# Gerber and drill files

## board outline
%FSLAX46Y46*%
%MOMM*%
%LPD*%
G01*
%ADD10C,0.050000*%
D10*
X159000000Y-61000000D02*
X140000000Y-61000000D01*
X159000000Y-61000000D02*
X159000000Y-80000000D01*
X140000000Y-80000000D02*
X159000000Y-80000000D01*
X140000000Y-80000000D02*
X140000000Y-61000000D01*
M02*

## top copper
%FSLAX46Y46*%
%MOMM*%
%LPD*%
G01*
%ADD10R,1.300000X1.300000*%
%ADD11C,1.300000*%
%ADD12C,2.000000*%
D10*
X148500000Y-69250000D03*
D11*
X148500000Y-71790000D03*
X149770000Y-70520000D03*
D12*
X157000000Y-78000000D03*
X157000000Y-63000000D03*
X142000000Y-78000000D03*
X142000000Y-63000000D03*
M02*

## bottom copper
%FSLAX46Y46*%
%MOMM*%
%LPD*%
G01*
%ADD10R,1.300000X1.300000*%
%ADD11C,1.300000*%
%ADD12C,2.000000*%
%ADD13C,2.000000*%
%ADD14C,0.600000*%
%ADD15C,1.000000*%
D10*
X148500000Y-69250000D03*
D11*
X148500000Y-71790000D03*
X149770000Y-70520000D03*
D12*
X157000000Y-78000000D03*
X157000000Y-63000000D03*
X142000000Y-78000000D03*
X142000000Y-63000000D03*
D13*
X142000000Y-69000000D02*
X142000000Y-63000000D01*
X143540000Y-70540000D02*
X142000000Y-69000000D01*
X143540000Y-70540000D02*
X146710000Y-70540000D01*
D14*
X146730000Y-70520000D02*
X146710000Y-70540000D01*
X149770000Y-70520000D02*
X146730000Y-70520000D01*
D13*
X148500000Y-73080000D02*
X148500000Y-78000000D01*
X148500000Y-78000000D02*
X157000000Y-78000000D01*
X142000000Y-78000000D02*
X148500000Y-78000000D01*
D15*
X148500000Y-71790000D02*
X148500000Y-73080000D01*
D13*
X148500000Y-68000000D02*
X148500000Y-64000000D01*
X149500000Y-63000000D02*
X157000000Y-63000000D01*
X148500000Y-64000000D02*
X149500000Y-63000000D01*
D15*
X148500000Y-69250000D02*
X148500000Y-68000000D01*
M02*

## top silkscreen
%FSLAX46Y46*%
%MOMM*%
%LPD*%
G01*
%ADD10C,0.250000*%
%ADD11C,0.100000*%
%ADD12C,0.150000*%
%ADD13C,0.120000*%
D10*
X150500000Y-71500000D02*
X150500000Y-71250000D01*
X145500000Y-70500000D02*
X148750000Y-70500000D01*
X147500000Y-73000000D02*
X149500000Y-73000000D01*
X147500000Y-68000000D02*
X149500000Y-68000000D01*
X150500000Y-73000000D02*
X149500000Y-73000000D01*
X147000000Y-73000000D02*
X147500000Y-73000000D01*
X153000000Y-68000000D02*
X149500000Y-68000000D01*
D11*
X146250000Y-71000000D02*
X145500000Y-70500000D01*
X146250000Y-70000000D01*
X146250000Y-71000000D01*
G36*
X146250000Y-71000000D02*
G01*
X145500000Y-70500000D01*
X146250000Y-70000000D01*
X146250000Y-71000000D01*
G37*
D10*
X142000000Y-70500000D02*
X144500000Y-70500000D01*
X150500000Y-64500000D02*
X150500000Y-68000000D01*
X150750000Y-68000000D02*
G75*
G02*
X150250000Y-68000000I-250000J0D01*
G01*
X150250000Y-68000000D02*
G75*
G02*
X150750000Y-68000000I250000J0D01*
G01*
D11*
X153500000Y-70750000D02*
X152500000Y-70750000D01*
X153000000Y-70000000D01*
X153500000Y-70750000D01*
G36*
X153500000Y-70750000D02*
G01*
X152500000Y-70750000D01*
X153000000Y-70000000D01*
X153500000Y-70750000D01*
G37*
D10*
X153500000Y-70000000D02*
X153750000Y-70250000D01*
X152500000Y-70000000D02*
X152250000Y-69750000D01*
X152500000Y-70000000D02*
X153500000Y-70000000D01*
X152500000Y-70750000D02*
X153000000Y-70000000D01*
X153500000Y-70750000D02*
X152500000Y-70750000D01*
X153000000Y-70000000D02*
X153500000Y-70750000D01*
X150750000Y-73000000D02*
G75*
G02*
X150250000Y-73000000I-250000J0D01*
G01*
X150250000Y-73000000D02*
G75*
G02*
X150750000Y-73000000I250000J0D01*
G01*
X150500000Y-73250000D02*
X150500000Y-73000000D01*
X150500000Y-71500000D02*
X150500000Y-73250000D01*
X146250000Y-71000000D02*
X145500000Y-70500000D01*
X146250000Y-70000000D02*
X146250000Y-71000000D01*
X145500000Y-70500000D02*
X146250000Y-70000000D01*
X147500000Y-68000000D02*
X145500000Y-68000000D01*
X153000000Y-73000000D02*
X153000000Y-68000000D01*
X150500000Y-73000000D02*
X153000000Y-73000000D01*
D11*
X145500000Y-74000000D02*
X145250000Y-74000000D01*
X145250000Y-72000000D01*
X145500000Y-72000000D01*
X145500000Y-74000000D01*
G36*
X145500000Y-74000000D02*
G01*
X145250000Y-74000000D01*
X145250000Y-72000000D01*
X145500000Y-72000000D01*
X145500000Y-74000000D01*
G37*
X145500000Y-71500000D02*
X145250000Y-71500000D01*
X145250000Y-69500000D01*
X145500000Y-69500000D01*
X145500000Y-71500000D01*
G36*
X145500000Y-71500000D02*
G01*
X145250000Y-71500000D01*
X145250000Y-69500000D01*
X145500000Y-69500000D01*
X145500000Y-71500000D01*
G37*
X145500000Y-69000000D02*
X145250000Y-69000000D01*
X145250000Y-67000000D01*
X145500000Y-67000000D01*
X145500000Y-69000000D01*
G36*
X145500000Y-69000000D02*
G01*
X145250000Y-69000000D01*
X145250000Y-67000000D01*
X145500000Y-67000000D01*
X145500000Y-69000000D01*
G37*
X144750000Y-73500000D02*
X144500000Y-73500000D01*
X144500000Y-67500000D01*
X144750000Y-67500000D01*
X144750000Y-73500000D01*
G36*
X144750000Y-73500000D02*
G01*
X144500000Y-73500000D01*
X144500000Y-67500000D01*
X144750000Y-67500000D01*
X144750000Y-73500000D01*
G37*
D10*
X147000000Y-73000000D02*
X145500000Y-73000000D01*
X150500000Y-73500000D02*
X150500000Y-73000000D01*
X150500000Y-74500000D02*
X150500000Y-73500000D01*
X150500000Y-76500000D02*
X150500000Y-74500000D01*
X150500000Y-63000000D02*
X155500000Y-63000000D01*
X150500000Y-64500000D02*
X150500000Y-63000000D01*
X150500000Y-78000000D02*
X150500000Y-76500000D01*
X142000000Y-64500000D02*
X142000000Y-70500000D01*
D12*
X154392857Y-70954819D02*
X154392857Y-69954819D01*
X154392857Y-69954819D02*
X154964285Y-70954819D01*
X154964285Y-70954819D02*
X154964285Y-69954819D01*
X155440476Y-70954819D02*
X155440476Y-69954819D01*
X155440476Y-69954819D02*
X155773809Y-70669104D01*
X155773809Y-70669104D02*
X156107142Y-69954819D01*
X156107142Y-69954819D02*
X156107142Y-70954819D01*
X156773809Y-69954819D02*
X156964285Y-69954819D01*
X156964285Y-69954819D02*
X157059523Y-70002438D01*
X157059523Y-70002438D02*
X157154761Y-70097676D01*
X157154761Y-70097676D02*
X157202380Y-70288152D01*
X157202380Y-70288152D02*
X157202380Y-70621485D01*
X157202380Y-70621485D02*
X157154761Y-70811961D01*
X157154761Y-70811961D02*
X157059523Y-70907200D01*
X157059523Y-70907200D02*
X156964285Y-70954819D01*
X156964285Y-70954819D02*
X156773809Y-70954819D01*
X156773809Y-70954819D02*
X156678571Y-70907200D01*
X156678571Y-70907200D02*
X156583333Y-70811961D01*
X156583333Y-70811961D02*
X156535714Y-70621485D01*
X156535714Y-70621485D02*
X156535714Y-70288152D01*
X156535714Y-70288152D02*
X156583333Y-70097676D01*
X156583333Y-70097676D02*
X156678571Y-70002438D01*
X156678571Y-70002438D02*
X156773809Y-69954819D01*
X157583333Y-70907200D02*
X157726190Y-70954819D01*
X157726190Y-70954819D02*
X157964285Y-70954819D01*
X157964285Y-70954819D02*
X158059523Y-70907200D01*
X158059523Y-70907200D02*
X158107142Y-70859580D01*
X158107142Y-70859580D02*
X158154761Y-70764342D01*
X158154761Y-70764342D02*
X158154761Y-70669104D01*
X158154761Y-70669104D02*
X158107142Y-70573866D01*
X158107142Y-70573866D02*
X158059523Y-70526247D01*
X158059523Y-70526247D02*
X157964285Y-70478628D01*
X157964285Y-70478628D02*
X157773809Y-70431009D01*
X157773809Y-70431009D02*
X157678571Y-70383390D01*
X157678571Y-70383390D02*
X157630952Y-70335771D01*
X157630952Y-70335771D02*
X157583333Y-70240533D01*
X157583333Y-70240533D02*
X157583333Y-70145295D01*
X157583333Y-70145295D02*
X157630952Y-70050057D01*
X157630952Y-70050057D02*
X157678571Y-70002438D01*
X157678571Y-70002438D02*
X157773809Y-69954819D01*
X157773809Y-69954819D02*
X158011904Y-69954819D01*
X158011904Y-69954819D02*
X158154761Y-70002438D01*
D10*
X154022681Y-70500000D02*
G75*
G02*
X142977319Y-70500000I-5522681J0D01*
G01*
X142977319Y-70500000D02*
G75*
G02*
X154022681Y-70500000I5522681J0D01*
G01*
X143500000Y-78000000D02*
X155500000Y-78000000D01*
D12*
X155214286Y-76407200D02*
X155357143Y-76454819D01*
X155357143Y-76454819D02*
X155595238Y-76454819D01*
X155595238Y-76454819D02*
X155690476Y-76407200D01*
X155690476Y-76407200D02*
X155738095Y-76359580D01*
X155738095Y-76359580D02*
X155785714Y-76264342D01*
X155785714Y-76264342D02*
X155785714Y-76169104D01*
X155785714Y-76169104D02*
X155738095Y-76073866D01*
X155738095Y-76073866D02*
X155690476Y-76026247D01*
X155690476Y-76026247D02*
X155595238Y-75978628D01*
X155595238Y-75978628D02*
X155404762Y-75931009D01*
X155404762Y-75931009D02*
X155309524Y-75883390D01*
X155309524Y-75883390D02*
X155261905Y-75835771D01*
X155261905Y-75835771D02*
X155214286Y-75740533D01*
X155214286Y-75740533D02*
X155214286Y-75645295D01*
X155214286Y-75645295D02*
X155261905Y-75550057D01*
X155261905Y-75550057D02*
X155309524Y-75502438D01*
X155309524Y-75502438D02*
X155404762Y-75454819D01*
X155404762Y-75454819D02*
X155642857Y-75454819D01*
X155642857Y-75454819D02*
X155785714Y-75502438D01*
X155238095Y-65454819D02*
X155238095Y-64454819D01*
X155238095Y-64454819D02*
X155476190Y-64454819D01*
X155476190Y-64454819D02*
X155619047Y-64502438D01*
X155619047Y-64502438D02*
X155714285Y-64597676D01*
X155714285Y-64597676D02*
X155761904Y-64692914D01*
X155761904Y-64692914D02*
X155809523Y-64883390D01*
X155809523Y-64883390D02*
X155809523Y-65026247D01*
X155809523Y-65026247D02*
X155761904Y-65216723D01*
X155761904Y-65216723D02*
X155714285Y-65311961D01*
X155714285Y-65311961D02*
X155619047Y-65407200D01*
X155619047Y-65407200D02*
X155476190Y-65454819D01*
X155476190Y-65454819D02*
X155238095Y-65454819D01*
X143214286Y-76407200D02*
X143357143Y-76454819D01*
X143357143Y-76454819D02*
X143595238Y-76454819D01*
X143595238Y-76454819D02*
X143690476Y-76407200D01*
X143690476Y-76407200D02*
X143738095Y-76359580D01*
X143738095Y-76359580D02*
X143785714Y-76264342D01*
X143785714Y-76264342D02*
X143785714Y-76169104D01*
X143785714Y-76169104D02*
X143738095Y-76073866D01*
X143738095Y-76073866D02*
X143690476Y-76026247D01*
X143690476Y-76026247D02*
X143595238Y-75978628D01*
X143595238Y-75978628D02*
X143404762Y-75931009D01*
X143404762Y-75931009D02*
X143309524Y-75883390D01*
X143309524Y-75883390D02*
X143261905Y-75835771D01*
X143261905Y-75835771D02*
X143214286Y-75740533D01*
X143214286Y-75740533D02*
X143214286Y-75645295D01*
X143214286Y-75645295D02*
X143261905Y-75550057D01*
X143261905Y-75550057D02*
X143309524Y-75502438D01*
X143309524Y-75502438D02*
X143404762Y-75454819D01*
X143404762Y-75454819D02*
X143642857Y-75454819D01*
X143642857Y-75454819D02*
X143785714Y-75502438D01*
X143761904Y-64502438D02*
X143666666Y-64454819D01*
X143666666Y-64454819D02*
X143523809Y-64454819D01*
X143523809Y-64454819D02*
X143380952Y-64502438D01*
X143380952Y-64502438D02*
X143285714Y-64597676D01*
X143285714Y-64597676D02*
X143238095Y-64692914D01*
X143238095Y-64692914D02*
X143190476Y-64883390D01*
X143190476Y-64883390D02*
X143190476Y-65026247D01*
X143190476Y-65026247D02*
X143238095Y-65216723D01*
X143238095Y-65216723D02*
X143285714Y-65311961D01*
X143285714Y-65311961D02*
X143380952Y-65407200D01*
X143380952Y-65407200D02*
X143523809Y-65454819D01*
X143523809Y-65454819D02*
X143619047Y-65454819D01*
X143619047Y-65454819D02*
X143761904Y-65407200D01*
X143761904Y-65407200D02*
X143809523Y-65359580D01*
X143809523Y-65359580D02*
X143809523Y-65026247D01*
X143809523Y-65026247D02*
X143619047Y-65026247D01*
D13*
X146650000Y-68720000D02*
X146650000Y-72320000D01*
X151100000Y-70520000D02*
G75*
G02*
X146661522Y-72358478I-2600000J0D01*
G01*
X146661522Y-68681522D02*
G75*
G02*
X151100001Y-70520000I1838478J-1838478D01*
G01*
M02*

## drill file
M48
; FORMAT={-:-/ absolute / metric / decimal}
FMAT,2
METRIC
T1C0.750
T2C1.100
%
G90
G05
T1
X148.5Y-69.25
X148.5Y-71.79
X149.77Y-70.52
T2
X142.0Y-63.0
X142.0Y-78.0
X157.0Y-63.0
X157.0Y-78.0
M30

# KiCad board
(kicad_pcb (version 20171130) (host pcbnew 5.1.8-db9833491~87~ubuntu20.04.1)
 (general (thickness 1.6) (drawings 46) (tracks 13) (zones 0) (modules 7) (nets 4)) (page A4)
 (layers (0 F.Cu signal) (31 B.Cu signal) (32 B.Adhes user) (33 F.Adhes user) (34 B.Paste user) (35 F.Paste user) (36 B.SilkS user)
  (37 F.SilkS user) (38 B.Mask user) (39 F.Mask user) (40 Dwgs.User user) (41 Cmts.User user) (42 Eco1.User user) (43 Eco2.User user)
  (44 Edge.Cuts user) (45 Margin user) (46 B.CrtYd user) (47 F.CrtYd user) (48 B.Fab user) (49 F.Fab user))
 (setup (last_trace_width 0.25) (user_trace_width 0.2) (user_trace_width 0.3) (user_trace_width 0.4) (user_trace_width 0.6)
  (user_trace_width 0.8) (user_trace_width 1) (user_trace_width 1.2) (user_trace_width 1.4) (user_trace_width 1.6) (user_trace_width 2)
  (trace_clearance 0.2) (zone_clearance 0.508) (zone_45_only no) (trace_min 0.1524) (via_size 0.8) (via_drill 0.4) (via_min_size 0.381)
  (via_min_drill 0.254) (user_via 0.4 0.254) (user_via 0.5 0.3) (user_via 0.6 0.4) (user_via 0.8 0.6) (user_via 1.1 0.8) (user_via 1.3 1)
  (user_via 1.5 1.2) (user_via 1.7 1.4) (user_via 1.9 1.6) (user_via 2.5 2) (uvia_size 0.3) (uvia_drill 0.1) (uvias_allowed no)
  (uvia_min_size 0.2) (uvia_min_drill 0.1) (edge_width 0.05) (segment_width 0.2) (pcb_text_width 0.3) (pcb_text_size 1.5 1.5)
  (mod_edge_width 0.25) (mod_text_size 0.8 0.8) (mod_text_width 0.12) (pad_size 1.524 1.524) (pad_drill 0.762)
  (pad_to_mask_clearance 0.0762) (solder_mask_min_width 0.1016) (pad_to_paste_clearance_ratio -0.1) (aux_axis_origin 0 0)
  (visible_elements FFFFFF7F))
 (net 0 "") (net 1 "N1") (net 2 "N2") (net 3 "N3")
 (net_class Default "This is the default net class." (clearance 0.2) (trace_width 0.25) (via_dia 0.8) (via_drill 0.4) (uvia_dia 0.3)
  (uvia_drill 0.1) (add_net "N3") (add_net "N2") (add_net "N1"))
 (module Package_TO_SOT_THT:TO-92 (layer F.Cu) (at 148.5 69.25 270)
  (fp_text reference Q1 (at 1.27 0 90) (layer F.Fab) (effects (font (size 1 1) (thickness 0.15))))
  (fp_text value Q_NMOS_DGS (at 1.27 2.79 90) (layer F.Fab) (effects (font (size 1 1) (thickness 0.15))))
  (fp_line (start -0.53 1.85) (end 3.07 1.85) (layer F.SilkS) (width 0.12))
  (fp_arc (start 1.27 0) (end 1.27 -2.6) (angle 135) (layer F.SilkS) (width 0.12))
  (fp_arc (start 1.27 0) (end 1.27 -2.6) (angle -135) (layer F.SilkS) (width 0.12))
  (pad 1 thru_hole rect (at 0 0 270) (size 1.3 1.3) (drill 0.75) (layers *.Cu *.Mask) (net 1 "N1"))
  (pad 3 thru_hole circle (at 2.54 0 270) (size 1.3 1.3) (drill 0.75) (layers *.Cu *.Mask) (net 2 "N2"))
  (pad 2 thru_hole circle (at 1.27 -1.27 270) (size 1.3 1.3) (drill 0.75) (layers *.Cu *.Mask) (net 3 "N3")))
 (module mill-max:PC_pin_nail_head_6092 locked (layer F.Cu) (at 157 78)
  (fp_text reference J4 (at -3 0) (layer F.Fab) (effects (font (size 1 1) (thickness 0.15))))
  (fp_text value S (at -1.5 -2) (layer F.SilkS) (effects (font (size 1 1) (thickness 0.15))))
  (pad 1 thru_hole circle (at 0 0) (size 2 2) (drill 1.1) (layers *.Cu *.Mask) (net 2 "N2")))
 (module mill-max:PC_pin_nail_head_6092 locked (layer F.Cu) (at 157 63)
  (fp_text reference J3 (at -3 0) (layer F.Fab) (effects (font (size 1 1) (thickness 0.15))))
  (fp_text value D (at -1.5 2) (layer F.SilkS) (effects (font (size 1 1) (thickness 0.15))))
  (pad 1 thru_hole circle (at 0 0) (size 2 2) (drill 1.1) (layers *.Cu *.Mask) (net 1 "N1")))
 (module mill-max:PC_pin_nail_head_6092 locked (layer F.Cu) (at 142 78)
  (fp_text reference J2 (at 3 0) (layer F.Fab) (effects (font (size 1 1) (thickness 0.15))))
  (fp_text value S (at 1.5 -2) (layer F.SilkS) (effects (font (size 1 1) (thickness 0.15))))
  (pad 1 thru_hole circle (at 0 0) (size 2 2) (drill 1.1) (layers *.Cu *.Mask) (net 2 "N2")))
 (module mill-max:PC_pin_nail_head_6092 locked (layer F.Cu) (at 142 63)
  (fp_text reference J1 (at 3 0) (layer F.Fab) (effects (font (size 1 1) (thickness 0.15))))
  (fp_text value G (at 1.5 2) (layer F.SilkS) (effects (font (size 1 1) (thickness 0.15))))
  (pad 1 thru_hole circle (at 0 0) (size 2 2) (drill 1.1) (layers *.Cu *.Mask) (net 3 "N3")))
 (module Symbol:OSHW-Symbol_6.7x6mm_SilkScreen (layer B.Cu) (at 153.75 70.5 270)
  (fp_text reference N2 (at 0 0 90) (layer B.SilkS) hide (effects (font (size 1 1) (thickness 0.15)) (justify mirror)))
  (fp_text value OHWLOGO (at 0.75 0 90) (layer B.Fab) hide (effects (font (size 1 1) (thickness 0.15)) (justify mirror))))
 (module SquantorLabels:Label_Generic (layer B.Cu) (at 157.75 71.5 90)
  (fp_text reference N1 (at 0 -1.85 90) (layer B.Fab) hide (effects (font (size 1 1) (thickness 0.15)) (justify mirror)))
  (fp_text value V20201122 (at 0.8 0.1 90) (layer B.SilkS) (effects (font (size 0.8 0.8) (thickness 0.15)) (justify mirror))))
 (gr_line (start 150.5 71.5) (end 150.5 71.25) (layer F.SilkS) (width 0.25))
 (gr_line (start 145.5 70.5) (end 148.75 70.5) (layer F.SilkS) (width 0.25))
 (gr_line (start 147.5 73) (end 149.5 73) (layer F.SilkS) (width 0.25))
 (gr_line (start 147.5 68) (end 149.5 68) (layer F.SilkS) (width 0.25))
 (gr_line (start 150.5 73) (end 149.5 73) (layer F.SilkS) (width 0.25))
 (gr_line (start 147 73) (end 147.5 73) (layer F.SilkS) (width 0.25))
 (gr_line (start 153 68) (end 149.5 68) (layer F.SilkS) (width 0.25))
 (gr_poly (pts (xy 146.25 71) (xy 145.5 70.5) (xy 146.25 70)) (layer F.SilkS) (width 0.1))
 (gr_line (start 142 70.5) (end 144.5 70.5) (layer F.SilkS) (width 0.25))
 (gr_line (start 150.5 64.5) (end 150.5 68) (layer F.SilkS) (width 0.25))
 (gr_circle (center 150.5 68) (end 150.75 68) (layer F.SilkS) (width 0.25))
 (gr_poly (pts (xy 153.5 70.75) (xy 152.5 70.75) (xy 153 70)) (layer F.SilkS) (width 0.1))
 (gr_line (start 153.5 70) (end 153.75 70.25) (layer F.SilkS) (width 0.25))
 (gr_line (start 152.5 70) (end 152.25 69.75) (layer F.SilkS) (width 0.25))
 (gr_line (start 152.5 70) (end 153.5 70) (layer F.SilkS) (width 0.25))
 (gr_line (start 152.5 70.75) (end 153 70) (layer F.SilkS) (width 0.25))
 (gr_line (start 153.5 70.75) (end 152.5 70.75) (layer F.SilkS) (width 0.25))
 (gr_line (start 153 70) (end 153.5 70.75) (layer F.SilkS) (width 0.25))
 (gr_circle (center 150.5 73) (end 150.75 73) (layer F.SilkS) (width 0.25))
 (gr_line (start 150.5 73.25) (end 150.5 73) (layer F.SilkS) (width 0.25))
 (gr_line (start 150.5 71.5) (end 150.5 73.25) (layer F.SilkS) (width 0.25))
 (gr_line (start 146.25 71) (end 145.5 70.5) (layer F.SilkS) (width 0.25))
 (gr_line (start 146.25 70) (end 146.25 71) (layer F.SilkS) (width 0.25))
 (gr_line (start 145.5 70.5) (end 146.25 70) (layer F.SilkS) (width 0.25))
 (gr_line (start 147.5 68) (end 145.5 68) (layer F.SilkS) (width 0.25))
 (gr_line (start 153 73) (end 153 68) (layer F.SilkS) (width 0.25))
 (gr_line (start 150.5 73) (end 153 73) (layer F.SilkS) (width 0.25))
 (gr_poly (pts (xy 145.5 74) (xy 145.25 74) (xy 145.25 72) (xy 145.5 72)) (layer F.SilkS) (width 0.1))
 (gr_poly (pts (xy 145.5 71.5) (xy 145.25 71.5) (xy 145.25 69.5) (xy 145.5 69.5)) (layer F.SilkS) (width 0.1))
 (gr_poly (pts (xy 145.5 69) (xy 145.25 69) (xy 145.25 67) (xy 145.5 67)) (layer F.SilkS) (width 0.1))
 (gr_poly (pts (xy 144.75 73.5) (xy 144.5 73.5) (xy 144.5 67.5) (xy 144.75 67.5)) (layer F.SilkS) (width 0.1))
 (gr_line (start 147 73) (end 145.5 73) (layer F.SilkS) (width 0.25))
 (gr_line (start 150.5 73.5) (end 150.5 73) (layer F.SilkS) (width 0.25))
 (gr_line (start 150.5 74.5) (end 150.5 73.5) (layer F.SilkS) (width 0.25))
 (gr_line (start 150.5 76.5) (end 150.5 74.5) (layer F.SilkS) (width 0.25))
 (gr_line (start 150.5 63) (end 155.5 63) (layer F.SilkS) (width 0.25))
 (gr_line (start 150.5 64.5) (end 150.5 63) (layer F.SilkS) (width 0.25))
 (gr_line (start 150.5 78) (end 150.5 76.5) (layer F.SilkS) (width 0.25))
 (gr_line (start 142 64.5) (end 142 70.5) (layer F.SilkS) (width 0.25))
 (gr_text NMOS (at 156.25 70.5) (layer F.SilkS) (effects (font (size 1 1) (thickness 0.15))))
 (gr_circle (center 148.5 70.5) (end 154 71) (layer F.SilkS) (width 0.25))
 (gr_line (start 143.5 78) (end 155.5 78) (layer F.SilkS) (width 0.25))
 (gr_line (start 159 61) (end 140 61) (layer Edge.Cuts) (width 0.05))
 (gr_line (start 159 61) (end 159 80) (layer Edge.Cuts) (width 0.05))
 (gr_line (start 140 80) (end 159 80) (layer Edge.Cuts) (width 0.05))
 (gr_line (start 140 80) (end 140 61) (layer Edge.Cuts) (width 0.05))
 (segment (start 142 69) (end 142 63) (width 2) (layer B.Cu) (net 3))
 (segment (start 143.54 70.54) (end 142 69) (width 2) (layer B.Cu) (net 3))
 (segment (start 143.54 70.54) (end 146.71 70.54) (width 2) (layer B.Cu) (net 3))
 (segment (start 146.73 70.52) (end 146.71 70.54) (width 0.6) (layer B.Cu) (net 3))
 (segment (start 149.77 70.52) (end 146.73 70.52) (width 0.6) (layer B.Cu) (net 3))
 (segment (start 148.5 73.08) (end 148.5 78) (width 2) (layer B.Cu) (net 2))
 (segment (start 148.5 78) (end 157 78) (width 2) (layer B.Cu) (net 2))
 (segment (start 142 78) (end 148.5 78) (width 2) (layer B.Cu) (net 2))
 (segment (start 148.5 71.79) (end 148.5 73.08) (width 1) (layer B.Cu) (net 2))
 (segment (start 148.5 68) (end 148.5 64) (width 2) (layer B.Cu) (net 1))
 (segment (start 149.5 63) (end 157 63) (width 2) (layer B.Cu) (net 1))
 (segment (start 148.5 64) (end 149.5 63) (width 2) (layer B.Cu) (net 1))
 (segment (start 148.5 69.25) (end 148.5 68) (width 1) (layer B.Cu) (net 1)))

